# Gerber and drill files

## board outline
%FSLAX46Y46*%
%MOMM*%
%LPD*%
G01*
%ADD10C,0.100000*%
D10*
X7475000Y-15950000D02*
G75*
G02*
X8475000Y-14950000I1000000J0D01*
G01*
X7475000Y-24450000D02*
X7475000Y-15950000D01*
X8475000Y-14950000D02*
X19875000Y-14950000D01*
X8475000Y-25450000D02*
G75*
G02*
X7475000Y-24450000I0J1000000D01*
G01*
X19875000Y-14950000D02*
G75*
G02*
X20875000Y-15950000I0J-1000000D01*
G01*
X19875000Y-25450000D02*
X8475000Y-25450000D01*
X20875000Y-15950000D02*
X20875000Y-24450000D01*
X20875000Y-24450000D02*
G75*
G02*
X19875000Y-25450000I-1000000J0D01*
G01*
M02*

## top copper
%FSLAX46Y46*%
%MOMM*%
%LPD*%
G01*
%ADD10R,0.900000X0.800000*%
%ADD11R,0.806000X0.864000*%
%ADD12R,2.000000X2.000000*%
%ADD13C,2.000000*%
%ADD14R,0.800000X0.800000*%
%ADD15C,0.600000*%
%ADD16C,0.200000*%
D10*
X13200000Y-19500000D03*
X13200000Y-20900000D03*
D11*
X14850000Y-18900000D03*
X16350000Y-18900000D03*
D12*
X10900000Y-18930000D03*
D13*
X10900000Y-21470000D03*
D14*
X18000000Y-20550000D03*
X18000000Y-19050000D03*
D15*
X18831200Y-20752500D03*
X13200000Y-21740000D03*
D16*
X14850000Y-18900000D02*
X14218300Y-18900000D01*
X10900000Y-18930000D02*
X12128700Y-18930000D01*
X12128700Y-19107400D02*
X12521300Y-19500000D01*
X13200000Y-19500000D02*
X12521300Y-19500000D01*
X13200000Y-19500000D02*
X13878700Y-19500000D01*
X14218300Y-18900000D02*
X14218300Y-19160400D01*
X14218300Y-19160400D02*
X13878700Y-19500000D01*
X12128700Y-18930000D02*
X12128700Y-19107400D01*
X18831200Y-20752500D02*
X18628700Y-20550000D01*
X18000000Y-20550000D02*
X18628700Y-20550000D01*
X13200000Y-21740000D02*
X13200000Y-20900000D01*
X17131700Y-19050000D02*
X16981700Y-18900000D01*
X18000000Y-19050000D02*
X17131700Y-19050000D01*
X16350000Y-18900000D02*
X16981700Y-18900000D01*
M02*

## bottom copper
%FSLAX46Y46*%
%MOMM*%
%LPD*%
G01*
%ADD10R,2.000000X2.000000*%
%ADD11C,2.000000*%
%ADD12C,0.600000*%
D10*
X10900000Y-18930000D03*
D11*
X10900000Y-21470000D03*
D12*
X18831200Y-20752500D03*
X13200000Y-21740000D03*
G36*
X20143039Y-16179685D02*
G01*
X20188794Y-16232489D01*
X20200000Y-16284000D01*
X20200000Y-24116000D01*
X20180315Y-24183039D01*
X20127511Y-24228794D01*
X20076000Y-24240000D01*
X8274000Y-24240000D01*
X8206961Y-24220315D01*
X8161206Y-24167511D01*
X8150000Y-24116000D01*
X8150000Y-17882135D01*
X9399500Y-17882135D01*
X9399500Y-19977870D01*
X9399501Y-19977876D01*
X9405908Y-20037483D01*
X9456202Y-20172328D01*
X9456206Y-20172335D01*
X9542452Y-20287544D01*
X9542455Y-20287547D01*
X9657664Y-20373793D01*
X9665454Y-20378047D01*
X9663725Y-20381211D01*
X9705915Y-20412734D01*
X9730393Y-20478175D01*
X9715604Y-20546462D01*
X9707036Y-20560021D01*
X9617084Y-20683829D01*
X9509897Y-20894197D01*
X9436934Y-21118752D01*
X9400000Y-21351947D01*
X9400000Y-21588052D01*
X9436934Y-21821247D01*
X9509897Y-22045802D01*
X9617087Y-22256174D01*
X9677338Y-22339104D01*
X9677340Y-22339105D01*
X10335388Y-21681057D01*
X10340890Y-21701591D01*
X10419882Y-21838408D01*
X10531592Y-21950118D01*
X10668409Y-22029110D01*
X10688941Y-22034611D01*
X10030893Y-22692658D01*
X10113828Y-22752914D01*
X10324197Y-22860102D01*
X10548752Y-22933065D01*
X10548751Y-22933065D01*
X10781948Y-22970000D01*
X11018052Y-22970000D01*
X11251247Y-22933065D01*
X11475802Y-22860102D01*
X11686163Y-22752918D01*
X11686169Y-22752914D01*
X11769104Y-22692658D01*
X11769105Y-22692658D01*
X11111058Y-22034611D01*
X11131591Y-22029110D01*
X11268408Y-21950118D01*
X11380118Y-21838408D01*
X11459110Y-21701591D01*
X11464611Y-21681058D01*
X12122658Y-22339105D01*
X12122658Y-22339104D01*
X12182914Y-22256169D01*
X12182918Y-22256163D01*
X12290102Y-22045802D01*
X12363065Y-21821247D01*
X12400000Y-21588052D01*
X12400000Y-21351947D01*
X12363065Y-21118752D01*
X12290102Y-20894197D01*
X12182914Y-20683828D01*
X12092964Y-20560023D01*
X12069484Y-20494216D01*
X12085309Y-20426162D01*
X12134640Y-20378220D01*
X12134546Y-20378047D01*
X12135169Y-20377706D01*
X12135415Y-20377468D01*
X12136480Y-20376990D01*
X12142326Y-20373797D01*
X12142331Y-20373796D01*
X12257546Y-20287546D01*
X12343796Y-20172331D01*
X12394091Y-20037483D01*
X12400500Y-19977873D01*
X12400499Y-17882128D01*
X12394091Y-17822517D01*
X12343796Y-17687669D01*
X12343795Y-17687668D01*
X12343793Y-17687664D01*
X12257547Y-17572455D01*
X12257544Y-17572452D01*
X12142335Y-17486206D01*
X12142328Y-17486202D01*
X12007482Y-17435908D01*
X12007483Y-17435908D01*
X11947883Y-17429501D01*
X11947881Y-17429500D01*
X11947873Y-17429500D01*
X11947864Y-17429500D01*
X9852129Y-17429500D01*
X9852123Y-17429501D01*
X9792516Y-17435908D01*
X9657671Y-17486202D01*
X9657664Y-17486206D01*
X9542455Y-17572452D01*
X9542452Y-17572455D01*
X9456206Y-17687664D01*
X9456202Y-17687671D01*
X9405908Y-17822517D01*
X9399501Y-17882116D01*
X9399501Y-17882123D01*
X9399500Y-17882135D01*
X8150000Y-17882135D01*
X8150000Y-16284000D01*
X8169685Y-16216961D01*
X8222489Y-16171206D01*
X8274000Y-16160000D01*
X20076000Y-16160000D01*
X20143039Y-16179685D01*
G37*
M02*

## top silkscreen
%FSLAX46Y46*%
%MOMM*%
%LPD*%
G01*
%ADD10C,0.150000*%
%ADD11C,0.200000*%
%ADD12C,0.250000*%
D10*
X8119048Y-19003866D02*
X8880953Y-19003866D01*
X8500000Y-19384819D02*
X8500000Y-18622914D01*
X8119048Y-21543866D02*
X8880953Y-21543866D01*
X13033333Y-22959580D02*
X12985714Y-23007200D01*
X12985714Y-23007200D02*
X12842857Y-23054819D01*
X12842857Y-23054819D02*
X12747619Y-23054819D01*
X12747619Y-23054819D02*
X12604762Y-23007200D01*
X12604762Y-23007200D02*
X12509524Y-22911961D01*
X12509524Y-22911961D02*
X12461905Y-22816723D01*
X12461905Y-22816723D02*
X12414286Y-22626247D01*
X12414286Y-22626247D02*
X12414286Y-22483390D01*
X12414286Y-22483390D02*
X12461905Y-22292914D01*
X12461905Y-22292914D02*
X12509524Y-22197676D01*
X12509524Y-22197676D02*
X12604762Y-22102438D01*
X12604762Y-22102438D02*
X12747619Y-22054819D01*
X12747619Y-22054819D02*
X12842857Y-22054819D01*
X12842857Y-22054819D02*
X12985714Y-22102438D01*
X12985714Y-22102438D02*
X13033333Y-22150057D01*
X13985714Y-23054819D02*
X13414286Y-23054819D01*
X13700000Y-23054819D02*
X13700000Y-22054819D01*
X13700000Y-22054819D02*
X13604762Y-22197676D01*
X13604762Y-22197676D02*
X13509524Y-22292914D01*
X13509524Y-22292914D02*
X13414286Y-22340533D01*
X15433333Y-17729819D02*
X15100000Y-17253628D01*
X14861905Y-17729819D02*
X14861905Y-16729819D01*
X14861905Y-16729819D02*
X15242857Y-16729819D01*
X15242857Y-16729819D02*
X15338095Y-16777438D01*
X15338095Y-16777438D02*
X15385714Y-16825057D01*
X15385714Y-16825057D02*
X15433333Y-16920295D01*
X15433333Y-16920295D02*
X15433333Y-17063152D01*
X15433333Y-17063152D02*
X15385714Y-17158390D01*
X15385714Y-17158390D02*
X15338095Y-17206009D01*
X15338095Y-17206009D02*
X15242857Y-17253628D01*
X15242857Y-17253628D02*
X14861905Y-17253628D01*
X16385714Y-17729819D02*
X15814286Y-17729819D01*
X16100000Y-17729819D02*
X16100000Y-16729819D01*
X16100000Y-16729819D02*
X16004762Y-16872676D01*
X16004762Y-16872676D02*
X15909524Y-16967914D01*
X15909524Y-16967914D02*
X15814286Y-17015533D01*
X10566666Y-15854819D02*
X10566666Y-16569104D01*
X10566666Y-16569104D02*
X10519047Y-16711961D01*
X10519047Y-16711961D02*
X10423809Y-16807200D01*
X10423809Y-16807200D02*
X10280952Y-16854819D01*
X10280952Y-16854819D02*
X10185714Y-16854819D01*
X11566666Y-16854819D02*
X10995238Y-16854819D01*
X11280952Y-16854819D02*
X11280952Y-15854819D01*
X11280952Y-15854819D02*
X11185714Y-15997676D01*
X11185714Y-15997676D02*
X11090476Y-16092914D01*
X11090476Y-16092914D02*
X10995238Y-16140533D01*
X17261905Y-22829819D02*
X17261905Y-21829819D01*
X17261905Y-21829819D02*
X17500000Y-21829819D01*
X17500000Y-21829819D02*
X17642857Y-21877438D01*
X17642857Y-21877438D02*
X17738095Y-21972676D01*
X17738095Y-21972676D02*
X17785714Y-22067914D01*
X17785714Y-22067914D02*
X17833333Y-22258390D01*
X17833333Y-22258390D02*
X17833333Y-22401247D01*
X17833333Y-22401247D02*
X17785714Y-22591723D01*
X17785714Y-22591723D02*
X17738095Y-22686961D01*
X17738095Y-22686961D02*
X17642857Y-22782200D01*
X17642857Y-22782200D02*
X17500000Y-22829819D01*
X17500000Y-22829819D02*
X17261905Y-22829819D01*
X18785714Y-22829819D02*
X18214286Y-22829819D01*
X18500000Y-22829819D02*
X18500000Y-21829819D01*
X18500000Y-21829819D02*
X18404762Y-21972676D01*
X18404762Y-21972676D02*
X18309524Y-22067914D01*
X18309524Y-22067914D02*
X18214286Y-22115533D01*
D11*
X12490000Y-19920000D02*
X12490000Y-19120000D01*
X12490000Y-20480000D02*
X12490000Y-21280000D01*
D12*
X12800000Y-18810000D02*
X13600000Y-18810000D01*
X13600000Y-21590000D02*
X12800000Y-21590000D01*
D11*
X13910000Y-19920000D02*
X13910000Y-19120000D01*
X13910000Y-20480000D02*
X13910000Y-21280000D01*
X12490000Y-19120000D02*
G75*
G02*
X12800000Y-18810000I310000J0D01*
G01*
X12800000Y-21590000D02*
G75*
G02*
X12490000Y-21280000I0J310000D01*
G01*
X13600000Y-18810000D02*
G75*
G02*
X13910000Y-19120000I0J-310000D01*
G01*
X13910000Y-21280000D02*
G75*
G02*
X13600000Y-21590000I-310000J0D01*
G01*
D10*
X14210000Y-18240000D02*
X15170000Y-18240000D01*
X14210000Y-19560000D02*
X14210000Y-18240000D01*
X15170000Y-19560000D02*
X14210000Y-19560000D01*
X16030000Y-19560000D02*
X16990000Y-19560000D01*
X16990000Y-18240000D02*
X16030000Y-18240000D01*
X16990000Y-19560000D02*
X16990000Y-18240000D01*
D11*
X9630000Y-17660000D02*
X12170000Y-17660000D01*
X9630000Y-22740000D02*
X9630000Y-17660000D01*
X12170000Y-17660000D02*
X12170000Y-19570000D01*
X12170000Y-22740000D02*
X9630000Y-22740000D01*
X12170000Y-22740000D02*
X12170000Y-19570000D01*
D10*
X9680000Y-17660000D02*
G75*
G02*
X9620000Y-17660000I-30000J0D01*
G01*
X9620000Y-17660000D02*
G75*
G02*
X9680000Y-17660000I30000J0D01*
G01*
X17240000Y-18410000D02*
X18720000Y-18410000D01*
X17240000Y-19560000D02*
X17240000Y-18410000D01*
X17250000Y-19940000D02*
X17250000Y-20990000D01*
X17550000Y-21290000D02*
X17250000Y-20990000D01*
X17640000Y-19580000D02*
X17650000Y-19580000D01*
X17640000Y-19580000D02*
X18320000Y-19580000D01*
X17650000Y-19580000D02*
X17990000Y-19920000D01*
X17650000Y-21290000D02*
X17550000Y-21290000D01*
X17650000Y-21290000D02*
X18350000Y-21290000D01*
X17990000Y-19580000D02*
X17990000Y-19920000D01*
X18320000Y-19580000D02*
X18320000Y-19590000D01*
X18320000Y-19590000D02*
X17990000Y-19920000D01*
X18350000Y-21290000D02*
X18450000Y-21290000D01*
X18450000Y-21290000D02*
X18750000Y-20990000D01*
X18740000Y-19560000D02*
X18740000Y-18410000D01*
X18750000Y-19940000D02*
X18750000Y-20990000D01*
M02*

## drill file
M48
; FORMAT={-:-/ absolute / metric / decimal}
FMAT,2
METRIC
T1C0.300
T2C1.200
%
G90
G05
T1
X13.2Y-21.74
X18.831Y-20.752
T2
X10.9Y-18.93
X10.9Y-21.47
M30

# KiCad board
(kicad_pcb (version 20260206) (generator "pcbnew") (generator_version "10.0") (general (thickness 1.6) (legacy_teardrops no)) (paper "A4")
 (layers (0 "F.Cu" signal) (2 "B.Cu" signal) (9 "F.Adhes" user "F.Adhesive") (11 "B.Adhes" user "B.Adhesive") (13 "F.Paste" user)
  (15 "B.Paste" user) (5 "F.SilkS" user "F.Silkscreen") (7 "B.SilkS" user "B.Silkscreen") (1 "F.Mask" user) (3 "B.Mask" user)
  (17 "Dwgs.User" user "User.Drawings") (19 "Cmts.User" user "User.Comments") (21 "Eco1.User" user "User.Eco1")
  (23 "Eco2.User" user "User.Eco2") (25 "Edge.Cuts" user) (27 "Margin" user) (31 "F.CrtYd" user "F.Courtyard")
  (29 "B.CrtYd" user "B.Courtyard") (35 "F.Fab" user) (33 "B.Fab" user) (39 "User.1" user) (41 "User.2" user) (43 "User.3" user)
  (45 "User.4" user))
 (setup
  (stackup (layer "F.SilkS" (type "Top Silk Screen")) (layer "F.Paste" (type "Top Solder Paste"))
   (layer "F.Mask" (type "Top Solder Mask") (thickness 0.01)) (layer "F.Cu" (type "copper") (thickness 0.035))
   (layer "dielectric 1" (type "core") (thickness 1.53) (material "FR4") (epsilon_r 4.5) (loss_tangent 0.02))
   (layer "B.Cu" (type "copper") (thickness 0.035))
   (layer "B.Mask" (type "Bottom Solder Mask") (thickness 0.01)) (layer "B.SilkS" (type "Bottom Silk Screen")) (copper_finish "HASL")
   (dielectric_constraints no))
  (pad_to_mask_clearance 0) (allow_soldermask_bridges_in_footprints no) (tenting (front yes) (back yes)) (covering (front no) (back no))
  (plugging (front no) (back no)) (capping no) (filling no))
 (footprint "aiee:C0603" (layer "F.Cu") (at 13.2 20.2 -90)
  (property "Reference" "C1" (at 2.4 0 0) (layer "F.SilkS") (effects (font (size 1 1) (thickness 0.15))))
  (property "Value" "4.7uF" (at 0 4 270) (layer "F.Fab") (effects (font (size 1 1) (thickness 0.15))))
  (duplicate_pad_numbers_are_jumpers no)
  (fp_line (start -0.28 0.71) (end -1.08 0.71) (stroke (width 0.2) (type solid)) (layer "F.SilkS"))
  (fp_line (start 0.28 0.71) (end 1.08 0.71) (stroke (width 0.2) (type solid)) (layer "F.SilkS"))
  (fp_line (start -1.39 0.4) (end -1.39 -0.4) (stroke (width 0.25) (type solid)) (layer "F.SilkS"))
  (fp_line (start 1.39 -0.4) (end 1.39 0.4) (stroke (width 0.25) (type solid)) (layer "F.SilkS"))
  (fp_line (start -0.28 -0.71) (end -1.08 -0.71) (stroke (width 0.2) (type solid)) (layer "F.SilkS"))
  (fp_line (start 0.28 -0.71) (end 1.08 -0.71) (stroke (width 0.2) (type solid)) (layer "F.SilkS"))
  (fp_arc (start -1.08 0.71) (mid -1.299203 0.619203) (end -1.39 0.4) (stroke (width 0.2) (type solid)) (layer "F.SilkS"))
  (fp_arc (start 1.39 0.4) (mid 1.299203 0.619203) (end 1.08 0.71) (stroke (width 0.2) (type solid)) (layer "F.SilkS"))
  (fp_arc (start -1.39 -0.4) (mid -1.299203 -0.619203) (end -1.08 -0.71) (stroke (width 0.2) (type solid)) (layer "F.SilkS"))
  (fp_arc (start 1.08 -0.71) (mid 1.299203 -0.619203) (end 1.39 -0.4) (stroke (width 0.2) (type solid)) (layer "F.SilkS"))
  (pad "1" smd rect (at -0.7 0 270) (size 0.8 0.9) (layers "F.Cu" "F.Mask" "F.Paste") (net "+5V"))
  (pad "2" smd rect (at 0.7 0 270) (size 0.8 0.9) (layers "F.Cu" "F.Mask" "F.Paste") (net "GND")))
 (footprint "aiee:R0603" (layer "F.Cu") (at 15.6 18.9)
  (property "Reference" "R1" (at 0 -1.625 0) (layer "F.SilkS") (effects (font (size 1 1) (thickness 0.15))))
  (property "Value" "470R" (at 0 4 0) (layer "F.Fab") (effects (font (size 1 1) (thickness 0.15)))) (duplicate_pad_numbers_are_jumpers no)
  (fp_line (start -1.39 -0.66) (end -0.43 -0.66) (stroke (width 0.15) (type solid)) (layer "F.SilkS"))
  (fp_line (start -1.39 0.66) (end -1.39 -0.66) (stroke (width 0.15) (type solid)) (layer "F.SilkS"))
  (fp_line (start -0.43 0.66) (end -1.39 0.66) (stroke (width 0.15) (type solid)) (layer "F.SilkS"))
  (fp_line (start 0.43 0.66) (end 1.39 0.66) (stroke (width 0.15) (type solid)) (layer "F.SilkS"))
  (fp_line (start 1.39 -0.66) (end 0.43 -0.66) (stroke (width 0.15) (type solid)) (layer "F.SilkS"))
  (fp_line (start 1.39 0.66) (end 1.39 -0.66) (stroke (width 0.15) (type solid)) (layer "F.SilkS"))
  (pad "1" smd rect (at -0.75 0) (size 0.806 0.864) (layers "F.Cu" "F.Mask" "F.Paste") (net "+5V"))
  (pad "2" smd rect (at 0.75 0) (size 0.806 0.864) (layers "F.Cu" "F.Mask" "F.Paste") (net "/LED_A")))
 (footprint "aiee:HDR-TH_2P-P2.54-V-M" (layer "F.Cu") (at 10.9 20.2 -90)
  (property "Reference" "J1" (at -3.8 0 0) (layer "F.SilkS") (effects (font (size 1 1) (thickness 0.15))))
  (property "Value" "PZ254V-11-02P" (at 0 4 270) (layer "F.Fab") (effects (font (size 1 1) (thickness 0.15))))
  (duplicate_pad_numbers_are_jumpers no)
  (fp_line (start -2.54 1.27) (end -2.54 -1.27) (stroke (width 0.2) (type solid)) (layer "F.SilkS"))
  (fp_line (start 2.54 1.27) (end -2.54 1.27) (stroke (width 0.2) (type solid)) (layer "F.SilkS"))
  (fp_line (start -2.54 -1.27) (end -0.63 -1.27) (stroke (width 0.2) (type solid)) (layer "F.SilkS"))
  (fp_line (start 2.54 -1.27) (end 2.54 1.27) (stroke (width 0.2) (type solid)) (layer "F.SilkS"))
  (fp_line (start 2.54 -1.27) (end -0.63 -1.27) (stroke (width 0.2) (type solid)) (layer "F.SilkS"))
  (fp_circle (center -2.54 1.25) (end -2.51 1.25) (stroke (width 0.15) (type solid)) (fill no) (layer "F.SilkS"))
  (pad "1" thru_hole rect (at -1.27 0 270) (size 2 2) (drill 1.199998) (layers "*.Cu" "*.Mask") (remove_unused_layers no) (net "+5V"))
  (pad "2" thru_hole circle (at 1.27 0 270) (size 2 2) (drill 1.199998) (layers "*.Cu" "*.Mask") (remove_unused_layers no) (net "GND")))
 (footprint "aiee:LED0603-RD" (layer "F.Cu") (at 18 19.8 90)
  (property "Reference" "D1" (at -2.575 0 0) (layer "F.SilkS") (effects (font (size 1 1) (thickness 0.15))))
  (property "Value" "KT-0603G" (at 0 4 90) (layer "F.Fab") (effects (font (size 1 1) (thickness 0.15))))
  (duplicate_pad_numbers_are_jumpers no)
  (fp_line (start 1.39 -0.76) (end 1.39 0.72) (stroke (width 0.15) (type solid)) (layer "F.SilkS"))
  (fp_line (start 0.24 -0.76) (end 1.39 -0.76) (stroke (width 0.15) (type solid)) (layer "F.SilkS"))
  (fp_line (start -0.14 -0.75) (end -1.19 -0.75) (stroke (width 0.15) (type solid)) (layer "F.SilkS"))
  (fp_line (start -1.49 -0.45) (end -1.19 -0.75) (stroke (width 0.15) (type solid)) (layer "F.SilkS"))
  (fp_line (start 0.22 -0.36) (end 0.22 -0.35) (stroke (width 0.15) (type solid)) (layer "F.SilkS"))
  (fp_line (start 0.22 -0.36) (end 0.22 0.32) (stroke (width 0.15) (type solid)) (layer "F.SilkS"))
  (fp_line (start 0.22 -0.35) (end -0.12 -0.01) (stroke (width 0.15) (type solid)) (layer "F.SilkS"))
  (fp_line (start -1.49 -0.35) (end -1.49 -0.45) (stroke (width 0.15) (type solid)) (layer "F.SilkS"))
  (fp_line (start -1.49 -0.35) (end -1.49 0.35) (stroke (width 0.15) (type solid)) (layer "F.SilkS"))
  (fp_line (start 0.22 -0.01) (end -0.12 -0.01) (stroke (width 0.15) (type solid)) (layer "F.SilkS"))
  (fp_line (start 0.22 0.32) (end 0.21 0.32) (stroke (width 0.15) (type solid)) (layer "F.SilkS"))
  (fp_line (start 0.21 0.32) (end -0.12 -0.01) (stroke (width 0.15) (type solid)) (layer "F.SilkS"))
  (fp_line (start -1.49 0.35) (end -1.49 0.45) (stroke (width 0.15) (type solid)) (layer "F.SilkS"))
  (fp_line (start -1.49 0.45) (end -1.19 0.75) (stroke (width 0.15) (type solid)) (layer "F.SilkS"))
  (fp_line (start 0.24 0.74) (end 1.39 0.74) (stroke (width 0.15) (type solid)) (layer "F.SilkS"))
  (fp_line (start -0.14 0.75) (end -1.19 0.75) (stroke (width 0.15) (type solid)) (layer "F.SilkS"))
  (pad "1" smd rect (at -0.75 0 180) (size 0.8 0.8) (layers "F.Cu" "F.Mask" "F.Paste") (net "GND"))
  (pad "2" smd rect (at 0.75 0 180) (size 0.8 0.8) (layers "F.Cu" "F.Mask" "F.Paste") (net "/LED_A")))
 (gr_arc (start 7.475 15.95) (mid 7.767893 15.242893) (end 8.475 14.95) (stroke (width 0.1) (type default)) (layer "Edge.Cuts"))
 (gr_line (start 7.475 24.45) (end 7.475 15.95) (stroke (width 0.1) (type default)) (layer "Edge.Cuts"))
 (gr_line (start 8.475 14.95) (end 19.875 14.95) (stroke (width 0.1) (type default)) (layer "Edge.Cuts"))
 (gr_arc (start 8.475 25.45) (mid 7.767893 25.157106) (end 7.475 24.45) (stroke (width 0.1) (type default)) (layer "Edge.Cuts"))
 (gr_arc (start 19.875 14.95) (mid 20.582106 15.242893) (end 20.875 15.95) (stroke (width 0.1) (type default)) (layer "Edge.Cuts"))
 (gr_line (start 19.875 25.45) (end 8.475 25.45) (stroke (width 0.1) (type default)) (layer "Edge.Cuts"))
 (gr_line (start 20.875 15.95) (end 20.875 24.45) (stroke (width 0.1) (type default)) (layer "Edge.Cuts"))
 (gr_arc (start 20.875 24.45) (mid 20.582106 25.157106) (end 19.875 25.45) (stroke (width 0.1) (type default)) (layer "Edge.Cuts"))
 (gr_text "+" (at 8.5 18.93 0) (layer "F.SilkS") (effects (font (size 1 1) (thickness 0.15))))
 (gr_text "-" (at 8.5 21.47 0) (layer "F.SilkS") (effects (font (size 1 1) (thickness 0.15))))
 (segment (start 14.85 18.9) (end 14.2183 18.9) (width 0.2) (layer "F.Cu") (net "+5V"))
 (segment (start 10.9 18.93) (end 12.1287 18.93) (width 0.2) (layer "F.Cu") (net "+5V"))
 (segment (start 12.1287 19.1074) (end 12.5213 19.5) (width 0.2) (layer "F.Cu") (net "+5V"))
 (segment (start 13.2 19.5) (end 12.5213 19.5) (width 0.2) (layer "F.Cu") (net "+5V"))
 (segment (start 13.2 19.5) (end 13.8787 19.5) (width 0.2) (layer "F.Cu") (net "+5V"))
 (segment (start 14.2183 18.9) (end 14.2183 19.1604) (width 0.2) (layer "F.Cu") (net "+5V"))
 (segment (start 14.2183 19.1604) (end 13.8787 19.5) (width 0.2) (layer "F.Cu") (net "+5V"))
 (segment (start 12.1287 18.93) (end 12.1287 19.1074) (width 0.2) (layer "F.Cu") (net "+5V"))
 (segment (start 18.8312 20.7525) (end 18.6287 20.55) (width 0.2) (layer "F.Cu") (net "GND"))
 (segment (start 18 20.55) (end 18.6287 20.55) (width 0.2) (layer "F.Cu") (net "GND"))
 (segment (start 13.2 21.74) (end 13.2 20.9) (width 0.2) (layer "F.Cu") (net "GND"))
 (via (at 18.8312 20.7525) (size 0.6) (drill 0.3) (layers "F.Cu" "B.Cu") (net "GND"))
 (via (at 13.2 21.74) (size 0.6) (drill 0.3) (layers "F.Cu" "B.Cu") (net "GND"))
 (segment (start 17.1317 19.05) (end 16.9817 18.9) (width 0.2) (layer "F.Cu") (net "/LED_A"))
 (segment (start 18 19.05) (end 17.1317 19.05) (width 0.2) (layer "F.Cu") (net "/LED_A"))
 (segment (start 16.35 18.9) (end 16.9817 18.9) (width 0.2) (layer "F.Cu") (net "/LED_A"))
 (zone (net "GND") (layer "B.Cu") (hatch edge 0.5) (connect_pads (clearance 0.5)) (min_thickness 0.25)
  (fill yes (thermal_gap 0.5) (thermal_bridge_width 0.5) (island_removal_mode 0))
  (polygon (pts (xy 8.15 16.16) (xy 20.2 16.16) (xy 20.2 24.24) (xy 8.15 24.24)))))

